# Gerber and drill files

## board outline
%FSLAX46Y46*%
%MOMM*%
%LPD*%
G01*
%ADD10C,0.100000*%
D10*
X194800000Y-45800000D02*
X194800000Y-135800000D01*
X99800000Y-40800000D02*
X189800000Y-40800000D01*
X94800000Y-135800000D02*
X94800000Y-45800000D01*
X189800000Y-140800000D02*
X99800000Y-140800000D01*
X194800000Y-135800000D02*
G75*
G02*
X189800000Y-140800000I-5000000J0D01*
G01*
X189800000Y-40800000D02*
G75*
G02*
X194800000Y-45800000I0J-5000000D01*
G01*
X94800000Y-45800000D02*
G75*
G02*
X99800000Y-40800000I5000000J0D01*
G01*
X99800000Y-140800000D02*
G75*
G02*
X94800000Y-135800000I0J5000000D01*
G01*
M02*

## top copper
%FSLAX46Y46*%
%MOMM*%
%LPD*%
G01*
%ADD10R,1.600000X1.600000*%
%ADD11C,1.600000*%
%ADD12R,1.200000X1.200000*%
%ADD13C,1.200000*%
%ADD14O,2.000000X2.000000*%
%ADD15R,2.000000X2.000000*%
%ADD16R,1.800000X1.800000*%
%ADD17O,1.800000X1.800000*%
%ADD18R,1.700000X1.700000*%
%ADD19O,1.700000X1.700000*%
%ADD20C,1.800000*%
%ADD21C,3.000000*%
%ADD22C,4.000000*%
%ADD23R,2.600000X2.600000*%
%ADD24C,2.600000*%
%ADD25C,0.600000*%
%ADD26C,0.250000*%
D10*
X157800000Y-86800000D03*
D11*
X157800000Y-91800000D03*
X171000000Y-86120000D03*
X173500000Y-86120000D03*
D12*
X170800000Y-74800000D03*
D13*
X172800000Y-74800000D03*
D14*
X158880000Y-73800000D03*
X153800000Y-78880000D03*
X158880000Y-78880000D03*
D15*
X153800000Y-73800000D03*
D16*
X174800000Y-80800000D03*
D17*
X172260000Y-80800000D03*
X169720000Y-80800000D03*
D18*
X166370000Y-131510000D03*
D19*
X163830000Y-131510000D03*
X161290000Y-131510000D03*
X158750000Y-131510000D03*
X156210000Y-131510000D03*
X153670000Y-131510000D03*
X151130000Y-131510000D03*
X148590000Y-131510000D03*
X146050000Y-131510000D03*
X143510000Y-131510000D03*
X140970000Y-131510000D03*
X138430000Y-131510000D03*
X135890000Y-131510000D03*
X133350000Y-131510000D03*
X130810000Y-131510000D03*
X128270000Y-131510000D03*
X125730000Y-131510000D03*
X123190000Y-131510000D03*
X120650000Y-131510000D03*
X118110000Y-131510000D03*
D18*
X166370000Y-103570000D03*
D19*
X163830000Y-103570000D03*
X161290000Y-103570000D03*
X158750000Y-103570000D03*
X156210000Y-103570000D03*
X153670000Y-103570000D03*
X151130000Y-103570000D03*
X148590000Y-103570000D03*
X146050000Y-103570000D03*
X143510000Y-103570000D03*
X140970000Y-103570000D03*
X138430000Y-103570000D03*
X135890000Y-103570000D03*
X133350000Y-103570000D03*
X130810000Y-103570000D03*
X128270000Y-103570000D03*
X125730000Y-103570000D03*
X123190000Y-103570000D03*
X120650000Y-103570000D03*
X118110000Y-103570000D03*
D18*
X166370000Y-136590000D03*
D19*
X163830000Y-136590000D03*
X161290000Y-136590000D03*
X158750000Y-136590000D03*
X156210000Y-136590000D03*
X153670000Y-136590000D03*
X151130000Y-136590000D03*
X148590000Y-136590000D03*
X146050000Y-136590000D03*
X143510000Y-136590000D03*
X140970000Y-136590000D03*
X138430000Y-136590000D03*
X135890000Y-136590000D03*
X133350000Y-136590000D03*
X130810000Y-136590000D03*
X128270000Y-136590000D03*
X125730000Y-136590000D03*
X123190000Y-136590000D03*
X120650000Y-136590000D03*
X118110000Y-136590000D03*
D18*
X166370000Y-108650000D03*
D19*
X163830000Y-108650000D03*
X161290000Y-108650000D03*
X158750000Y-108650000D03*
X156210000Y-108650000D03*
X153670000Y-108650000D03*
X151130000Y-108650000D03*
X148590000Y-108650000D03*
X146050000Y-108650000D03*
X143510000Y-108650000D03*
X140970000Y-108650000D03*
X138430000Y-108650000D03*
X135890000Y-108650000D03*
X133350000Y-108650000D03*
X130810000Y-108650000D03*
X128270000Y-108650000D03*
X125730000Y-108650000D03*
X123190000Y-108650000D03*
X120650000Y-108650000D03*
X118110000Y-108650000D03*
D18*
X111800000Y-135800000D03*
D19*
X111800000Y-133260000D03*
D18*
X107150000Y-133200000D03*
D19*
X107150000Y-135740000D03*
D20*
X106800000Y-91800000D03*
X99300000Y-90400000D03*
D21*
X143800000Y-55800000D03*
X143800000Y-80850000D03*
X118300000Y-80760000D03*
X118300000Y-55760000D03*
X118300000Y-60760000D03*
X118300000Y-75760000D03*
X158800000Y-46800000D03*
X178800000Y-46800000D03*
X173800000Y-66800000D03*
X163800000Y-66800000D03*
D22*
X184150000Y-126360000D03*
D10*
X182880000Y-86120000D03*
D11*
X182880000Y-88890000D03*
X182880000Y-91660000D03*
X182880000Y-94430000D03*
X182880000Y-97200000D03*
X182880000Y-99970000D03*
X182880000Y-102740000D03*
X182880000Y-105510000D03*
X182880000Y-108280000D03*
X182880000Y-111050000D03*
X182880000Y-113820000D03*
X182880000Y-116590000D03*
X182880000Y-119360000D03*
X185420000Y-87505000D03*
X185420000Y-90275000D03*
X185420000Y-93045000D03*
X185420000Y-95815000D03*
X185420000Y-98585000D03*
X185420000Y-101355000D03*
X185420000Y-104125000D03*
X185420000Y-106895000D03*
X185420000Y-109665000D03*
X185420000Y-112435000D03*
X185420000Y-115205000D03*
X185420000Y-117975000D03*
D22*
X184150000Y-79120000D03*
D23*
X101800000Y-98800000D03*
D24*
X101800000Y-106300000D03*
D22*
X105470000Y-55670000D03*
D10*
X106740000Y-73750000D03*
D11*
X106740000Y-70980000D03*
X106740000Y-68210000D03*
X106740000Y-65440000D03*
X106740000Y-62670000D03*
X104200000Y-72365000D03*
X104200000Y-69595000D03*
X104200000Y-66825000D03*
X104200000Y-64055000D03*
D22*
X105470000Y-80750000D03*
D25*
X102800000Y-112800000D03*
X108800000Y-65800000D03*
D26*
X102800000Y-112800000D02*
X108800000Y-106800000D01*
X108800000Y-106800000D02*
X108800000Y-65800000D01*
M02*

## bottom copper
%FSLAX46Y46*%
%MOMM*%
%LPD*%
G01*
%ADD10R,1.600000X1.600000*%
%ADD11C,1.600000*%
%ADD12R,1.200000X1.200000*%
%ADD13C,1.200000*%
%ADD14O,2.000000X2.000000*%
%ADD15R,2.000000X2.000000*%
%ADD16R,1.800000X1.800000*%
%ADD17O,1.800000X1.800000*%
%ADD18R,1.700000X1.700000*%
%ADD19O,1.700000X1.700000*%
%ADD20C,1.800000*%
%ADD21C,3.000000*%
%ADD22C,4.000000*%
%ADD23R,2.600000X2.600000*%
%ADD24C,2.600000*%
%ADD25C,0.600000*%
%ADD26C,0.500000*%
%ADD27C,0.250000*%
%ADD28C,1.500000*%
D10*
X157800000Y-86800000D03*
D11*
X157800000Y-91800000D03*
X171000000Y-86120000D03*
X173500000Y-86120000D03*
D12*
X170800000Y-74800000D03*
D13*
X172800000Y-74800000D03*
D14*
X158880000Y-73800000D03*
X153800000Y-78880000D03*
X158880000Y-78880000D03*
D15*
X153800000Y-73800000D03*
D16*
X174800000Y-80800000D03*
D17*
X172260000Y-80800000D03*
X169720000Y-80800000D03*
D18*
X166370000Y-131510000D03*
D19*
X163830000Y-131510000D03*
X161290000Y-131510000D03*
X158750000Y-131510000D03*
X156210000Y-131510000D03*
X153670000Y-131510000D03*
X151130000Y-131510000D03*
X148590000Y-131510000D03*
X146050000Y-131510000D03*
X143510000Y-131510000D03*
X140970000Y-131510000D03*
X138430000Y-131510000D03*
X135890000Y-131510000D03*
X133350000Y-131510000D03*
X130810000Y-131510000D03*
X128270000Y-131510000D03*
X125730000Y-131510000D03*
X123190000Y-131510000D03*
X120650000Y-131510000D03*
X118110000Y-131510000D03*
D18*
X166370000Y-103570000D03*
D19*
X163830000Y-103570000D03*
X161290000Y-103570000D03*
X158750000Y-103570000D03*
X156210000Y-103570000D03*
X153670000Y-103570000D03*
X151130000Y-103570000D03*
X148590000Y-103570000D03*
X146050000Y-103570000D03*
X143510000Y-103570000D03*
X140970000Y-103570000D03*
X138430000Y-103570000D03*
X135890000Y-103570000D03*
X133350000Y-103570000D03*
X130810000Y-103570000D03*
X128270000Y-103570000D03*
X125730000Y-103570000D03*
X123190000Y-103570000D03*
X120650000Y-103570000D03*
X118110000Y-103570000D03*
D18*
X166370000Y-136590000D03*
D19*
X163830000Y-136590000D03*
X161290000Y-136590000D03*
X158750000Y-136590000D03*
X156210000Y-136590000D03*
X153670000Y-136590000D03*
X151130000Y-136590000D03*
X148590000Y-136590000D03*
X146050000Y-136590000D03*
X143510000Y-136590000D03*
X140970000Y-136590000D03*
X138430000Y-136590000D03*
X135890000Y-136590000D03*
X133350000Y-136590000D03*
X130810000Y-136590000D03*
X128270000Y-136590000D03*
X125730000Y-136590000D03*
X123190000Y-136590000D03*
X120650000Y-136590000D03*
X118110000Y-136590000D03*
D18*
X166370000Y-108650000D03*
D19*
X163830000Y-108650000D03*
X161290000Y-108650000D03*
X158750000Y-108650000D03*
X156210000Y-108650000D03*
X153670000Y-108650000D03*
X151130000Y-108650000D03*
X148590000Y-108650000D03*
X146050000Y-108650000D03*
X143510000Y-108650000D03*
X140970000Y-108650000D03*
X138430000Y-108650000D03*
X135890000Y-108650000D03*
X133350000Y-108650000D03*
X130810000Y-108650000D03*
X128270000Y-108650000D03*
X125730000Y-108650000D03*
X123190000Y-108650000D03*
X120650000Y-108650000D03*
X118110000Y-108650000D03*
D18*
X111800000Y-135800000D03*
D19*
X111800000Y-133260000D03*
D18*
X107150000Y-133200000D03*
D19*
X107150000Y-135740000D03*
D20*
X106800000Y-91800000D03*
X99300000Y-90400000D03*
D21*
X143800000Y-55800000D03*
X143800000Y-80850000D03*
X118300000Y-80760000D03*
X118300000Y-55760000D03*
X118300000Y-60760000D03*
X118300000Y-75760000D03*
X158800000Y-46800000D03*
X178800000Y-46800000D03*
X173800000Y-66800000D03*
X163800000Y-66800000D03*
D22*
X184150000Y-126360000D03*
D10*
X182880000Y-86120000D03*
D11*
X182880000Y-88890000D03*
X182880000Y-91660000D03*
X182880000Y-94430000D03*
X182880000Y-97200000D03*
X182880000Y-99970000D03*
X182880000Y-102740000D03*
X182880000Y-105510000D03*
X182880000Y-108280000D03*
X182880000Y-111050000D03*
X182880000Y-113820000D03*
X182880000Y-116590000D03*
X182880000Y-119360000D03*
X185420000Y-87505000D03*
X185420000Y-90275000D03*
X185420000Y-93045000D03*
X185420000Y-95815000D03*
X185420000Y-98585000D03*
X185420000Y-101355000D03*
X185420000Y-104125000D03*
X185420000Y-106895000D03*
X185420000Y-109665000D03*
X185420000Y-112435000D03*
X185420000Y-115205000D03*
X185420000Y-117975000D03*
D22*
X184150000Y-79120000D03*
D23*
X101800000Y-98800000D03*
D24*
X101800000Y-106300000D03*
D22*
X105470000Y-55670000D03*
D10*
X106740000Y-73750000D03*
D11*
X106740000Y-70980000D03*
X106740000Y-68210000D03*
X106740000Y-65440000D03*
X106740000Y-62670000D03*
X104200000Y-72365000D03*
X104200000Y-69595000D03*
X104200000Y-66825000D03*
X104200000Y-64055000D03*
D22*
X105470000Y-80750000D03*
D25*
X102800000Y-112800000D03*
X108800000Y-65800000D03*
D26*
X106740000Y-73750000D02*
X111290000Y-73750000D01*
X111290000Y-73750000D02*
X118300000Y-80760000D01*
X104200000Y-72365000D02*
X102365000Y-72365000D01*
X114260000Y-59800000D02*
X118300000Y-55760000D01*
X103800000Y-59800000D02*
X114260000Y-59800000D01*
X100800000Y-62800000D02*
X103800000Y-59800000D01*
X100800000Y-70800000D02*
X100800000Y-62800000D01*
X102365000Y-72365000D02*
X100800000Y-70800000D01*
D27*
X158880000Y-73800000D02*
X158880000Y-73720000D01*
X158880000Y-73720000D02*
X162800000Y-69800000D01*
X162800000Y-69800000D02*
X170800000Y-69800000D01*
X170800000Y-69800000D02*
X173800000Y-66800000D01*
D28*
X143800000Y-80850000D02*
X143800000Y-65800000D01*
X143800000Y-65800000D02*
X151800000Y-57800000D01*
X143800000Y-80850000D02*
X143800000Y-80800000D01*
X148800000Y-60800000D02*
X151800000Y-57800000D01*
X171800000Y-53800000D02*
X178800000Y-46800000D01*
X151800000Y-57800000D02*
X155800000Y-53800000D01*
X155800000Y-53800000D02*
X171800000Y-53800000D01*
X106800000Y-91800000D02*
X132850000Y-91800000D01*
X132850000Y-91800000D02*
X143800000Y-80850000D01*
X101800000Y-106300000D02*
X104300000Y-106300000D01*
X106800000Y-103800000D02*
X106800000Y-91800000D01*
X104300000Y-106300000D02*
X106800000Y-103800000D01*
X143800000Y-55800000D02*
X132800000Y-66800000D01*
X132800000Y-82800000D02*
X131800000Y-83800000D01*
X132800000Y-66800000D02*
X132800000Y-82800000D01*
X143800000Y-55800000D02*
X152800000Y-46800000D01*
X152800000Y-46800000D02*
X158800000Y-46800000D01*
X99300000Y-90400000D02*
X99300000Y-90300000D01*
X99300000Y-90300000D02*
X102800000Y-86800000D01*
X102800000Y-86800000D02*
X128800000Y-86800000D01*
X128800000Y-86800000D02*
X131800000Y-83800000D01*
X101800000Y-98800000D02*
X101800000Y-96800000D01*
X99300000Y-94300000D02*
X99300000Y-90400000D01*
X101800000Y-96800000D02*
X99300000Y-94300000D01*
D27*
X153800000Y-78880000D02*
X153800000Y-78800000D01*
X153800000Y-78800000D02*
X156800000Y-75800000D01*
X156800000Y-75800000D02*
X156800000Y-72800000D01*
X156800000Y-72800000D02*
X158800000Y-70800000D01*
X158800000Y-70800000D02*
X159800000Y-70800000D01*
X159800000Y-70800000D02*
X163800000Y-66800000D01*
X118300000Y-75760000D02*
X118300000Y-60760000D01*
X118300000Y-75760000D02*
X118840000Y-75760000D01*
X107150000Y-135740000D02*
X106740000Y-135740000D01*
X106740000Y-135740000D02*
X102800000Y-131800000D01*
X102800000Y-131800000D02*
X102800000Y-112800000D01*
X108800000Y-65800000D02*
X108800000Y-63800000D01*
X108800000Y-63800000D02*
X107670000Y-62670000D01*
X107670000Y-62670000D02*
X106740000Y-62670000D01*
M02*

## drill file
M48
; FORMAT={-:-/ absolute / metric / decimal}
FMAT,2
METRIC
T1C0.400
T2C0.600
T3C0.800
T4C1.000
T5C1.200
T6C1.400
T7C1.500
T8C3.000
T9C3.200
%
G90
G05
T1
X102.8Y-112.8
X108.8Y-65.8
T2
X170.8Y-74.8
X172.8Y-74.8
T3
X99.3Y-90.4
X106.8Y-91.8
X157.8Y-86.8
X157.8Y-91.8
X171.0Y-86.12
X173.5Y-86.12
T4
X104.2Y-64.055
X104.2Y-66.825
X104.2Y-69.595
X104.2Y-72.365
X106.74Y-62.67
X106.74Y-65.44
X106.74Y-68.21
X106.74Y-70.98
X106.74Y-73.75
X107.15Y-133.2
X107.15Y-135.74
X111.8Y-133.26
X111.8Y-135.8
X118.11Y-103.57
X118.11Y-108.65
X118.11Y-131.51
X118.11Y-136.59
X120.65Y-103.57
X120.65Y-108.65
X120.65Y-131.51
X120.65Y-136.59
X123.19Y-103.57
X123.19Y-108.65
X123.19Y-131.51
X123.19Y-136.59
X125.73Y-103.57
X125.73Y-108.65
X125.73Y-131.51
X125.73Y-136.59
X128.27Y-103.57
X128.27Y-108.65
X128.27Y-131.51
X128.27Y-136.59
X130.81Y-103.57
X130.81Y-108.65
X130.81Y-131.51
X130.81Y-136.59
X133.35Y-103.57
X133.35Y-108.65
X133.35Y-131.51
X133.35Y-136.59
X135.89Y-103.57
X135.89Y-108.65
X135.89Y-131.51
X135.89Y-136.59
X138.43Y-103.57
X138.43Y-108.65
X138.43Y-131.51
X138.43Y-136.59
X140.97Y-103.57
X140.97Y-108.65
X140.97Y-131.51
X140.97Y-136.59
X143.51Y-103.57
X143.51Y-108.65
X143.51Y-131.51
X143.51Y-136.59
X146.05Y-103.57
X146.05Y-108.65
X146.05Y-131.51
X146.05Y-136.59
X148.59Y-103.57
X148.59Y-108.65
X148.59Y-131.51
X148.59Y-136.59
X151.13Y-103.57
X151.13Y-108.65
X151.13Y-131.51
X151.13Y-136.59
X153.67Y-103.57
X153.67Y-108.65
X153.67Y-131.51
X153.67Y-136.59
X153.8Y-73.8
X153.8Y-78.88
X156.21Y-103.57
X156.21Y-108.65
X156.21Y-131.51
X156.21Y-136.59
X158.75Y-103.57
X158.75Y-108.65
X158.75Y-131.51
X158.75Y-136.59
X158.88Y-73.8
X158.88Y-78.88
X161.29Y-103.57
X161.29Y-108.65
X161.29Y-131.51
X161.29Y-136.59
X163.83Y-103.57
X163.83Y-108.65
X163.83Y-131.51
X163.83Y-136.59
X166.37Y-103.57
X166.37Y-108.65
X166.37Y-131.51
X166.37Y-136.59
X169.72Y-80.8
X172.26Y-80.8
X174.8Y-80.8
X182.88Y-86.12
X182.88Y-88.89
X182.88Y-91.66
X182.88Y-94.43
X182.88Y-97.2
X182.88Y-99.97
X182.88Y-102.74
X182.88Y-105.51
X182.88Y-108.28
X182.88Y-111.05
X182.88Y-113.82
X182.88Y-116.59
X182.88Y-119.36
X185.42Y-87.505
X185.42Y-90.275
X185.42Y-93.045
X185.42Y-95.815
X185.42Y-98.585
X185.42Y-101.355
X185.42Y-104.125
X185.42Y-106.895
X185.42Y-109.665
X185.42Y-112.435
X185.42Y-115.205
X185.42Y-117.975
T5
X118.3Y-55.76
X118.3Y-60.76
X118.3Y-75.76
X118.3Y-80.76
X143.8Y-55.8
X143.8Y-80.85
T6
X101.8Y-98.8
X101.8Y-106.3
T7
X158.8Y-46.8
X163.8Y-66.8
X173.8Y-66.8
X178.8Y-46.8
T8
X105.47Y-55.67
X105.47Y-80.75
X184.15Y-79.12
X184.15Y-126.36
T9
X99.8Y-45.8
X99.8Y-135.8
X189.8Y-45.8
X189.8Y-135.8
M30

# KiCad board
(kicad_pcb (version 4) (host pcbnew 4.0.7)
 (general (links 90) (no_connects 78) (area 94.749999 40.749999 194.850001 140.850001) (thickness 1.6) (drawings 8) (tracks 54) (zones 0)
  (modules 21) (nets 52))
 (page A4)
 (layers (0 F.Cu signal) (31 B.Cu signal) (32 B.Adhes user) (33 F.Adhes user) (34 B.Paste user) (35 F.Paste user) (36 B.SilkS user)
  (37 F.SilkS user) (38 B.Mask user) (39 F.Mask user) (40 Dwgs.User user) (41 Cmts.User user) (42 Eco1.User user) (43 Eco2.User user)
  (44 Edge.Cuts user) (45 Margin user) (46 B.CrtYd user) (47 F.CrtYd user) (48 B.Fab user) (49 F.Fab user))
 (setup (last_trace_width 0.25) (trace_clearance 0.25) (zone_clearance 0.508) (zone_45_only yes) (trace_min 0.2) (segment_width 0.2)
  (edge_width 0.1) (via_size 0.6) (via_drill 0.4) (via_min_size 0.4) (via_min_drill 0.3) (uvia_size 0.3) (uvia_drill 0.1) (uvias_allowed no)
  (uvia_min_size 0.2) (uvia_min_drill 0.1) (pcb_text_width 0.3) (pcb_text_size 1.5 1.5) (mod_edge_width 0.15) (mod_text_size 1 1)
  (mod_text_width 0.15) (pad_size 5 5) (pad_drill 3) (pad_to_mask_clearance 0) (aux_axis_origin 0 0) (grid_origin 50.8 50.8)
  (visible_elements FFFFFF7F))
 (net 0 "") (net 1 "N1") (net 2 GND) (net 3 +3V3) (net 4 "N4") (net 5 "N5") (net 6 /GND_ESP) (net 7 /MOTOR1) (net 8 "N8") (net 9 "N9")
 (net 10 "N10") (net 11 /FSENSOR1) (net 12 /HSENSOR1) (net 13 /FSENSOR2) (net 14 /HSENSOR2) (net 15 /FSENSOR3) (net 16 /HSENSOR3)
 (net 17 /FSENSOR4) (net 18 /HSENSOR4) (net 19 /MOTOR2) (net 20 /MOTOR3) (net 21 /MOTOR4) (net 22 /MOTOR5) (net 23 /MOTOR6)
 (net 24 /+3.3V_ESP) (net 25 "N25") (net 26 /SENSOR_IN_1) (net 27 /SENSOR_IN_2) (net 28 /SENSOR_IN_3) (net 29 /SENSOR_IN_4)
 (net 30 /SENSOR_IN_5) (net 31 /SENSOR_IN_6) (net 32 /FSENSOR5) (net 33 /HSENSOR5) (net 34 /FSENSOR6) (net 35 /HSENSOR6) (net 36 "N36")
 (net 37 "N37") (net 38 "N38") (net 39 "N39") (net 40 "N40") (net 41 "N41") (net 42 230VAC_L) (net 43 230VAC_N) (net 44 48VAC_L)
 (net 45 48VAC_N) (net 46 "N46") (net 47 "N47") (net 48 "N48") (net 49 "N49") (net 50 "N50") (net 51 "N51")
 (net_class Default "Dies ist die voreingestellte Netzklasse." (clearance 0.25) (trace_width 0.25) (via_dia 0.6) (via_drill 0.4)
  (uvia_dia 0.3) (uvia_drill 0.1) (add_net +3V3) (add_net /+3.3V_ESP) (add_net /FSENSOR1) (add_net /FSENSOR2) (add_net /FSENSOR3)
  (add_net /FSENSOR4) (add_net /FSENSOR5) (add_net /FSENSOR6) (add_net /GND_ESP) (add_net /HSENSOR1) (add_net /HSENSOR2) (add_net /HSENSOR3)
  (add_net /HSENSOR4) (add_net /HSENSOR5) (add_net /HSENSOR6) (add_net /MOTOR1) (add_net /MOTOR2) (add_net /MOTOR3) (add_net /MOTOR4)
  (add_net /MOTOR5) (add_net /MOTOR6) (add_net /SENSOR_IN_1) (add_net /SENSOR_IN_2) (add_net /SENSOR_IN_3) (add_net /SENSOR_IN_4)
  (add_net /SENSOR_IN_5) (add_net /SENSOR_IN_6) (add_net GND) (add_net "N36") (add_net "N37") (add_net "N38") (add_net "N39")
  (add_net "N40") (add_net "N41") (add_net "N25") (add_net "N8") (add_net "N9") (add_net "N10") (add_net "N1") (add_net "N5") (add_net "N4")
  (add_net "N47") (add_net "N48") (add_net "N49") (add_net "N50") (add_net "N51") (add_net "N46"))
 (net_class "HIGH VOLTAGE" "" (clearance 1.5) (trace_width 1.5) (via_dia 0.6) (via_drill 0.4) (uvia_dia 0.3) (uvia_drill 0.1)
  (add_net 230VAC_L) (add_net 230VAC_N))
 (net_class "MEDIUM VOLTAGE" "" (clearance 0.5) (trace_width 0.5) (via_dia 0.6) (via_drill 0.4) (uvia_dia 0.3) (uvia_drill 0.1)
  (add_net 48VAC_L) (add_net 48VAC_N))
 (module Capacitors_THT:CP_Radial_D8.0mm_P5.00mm (layer F.Cu) (at 157.8 86.8 270)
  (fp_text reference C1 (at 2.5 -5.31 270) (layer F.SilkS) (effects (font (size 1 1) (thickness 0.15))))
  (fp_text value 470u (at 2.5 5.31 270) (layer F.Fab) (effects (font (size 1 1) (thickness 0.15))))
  (pad 1 thru_hole rect (at 0 0 270) (size 1.6 1.6) (drill 0.8) (layers *.Cu *.Mask) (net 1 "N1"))
  (pad 2 thru_hole circle (at 5 0 270) (size 1.6 1.6) (drill 0.8) (layers *.Cu *.Mask) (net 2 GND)))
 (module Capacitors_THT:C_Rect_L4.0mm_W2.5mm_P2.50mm (layer F.Cu) (at 171 86.12)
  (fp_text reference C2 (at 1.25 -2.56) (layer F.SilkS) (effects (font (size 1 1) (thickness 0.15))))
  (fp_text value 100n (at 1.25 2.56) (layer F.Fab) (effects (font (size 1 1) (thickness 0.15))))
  (pad 1 thru_hole circle (at 0 0) (size 1.6 1.6) (drill 0.8) (layers *.Cu *.Mask) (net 1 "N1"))
  (pad 2 thru_hole circle (at 2.5 0) (size 1.6 1.6) (drill 0.8) (layers *.Cu *.Mask) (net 2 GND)))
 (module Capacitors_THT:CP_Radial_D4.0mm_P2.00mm (layer F.Cu) (at 170.8 74.8)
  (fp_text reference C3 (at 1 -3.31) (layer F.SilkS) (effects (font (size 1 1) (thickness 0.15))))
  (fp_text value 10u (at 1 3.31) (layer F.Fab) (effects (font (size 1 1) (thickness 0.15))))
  (pad 1 thru_hole rect (at 0 0) (size 1.2 1.2) (drill 0.6) (layers *.Cu *.Mask) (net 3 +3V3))
  (pad 2 thru_hole circle (at 2 0) (size 1.2 1.2) (drill 0.6) (layers *.Cu *.Mask) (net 2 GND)))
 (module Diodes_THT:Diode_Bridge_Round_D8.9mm (layer F.Cu) (at 153.8 73.8)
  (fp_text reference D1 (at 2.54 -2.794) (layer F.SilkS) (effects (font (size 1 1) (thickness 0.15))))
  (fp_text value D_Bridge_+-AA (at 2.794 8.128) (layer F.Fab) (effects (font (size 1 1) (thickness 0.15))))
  (pad 4 thru_hole oval (at 5.08 0) (size 2 2) (drill 1) (layers *.Cu *.Mask) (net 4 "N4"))
  (pad 2 thru_hole oval (at 0 5.08) (size 2 2) (drill 1) (layers *.Cu *.Mask) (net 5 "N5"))
  (pad 3 thru_hole oval (at 5.08 5.08) (size 2 2) (drill 1) (layers *.Cu *.Mask) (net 2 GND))
  (pad 1 thru_hole rect (at 0 0) (size 2 2) (drill 1) (layers *.Cu *.Mask) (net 1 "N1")))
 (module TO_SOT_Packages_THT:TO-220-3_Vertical (layer F.Cu) (at 174.8 80.8 180)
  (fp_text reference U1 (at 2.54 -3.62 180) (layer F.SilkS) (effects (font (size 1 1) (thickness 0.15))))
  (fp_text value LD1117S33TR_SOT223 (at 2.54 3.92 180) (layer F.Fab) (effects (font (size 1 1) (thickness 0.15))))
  (pad 1 thru_hole rect (at 0 0 180) (size 1.8 1.8) (drill 1) (layers *.Cu *.Mask) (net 2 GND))
  (pad 2 thru_hole oval (at 2.54 0 180) (size 1.8 1.8) (drill 1) (layers *.Cu *.Mask) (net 3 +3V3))
  (pad 3 thru_hole oval (at 5.08 0 180) (size 1.8 1.8) (drill 1) (layers *.Cu *.Mask) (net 1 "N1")))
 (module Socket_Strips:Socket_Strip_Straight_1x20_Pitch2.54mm (layer F.Cu) (at 166.37 131.51 270)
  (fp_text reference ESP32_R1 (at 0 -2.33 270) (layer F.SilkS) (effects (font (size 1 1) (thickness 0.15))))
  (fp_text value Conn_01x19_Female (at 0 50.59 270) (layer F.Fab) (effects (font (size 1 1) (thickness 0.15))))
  (pad 1 thru_hole rect (at 0 0 270) (size 1.7 1.7) (drill 1) (layers *.Cu *.Mask) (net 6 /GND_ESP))
  (pad 2 thru_hole oval (at 0 2.54 270) (size 1.7 1.7) (drill 1) (layers *.Cu *.Mask) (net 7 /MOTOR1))
  (pad 3 thru_hole oval (at 0 5.08 270) (size 1.7 1.7) (drill 1) (layers *.Cu *.Mask) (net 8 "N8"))
  (pad 4 thru_hole oval (at 0 7.62 270) (size 1.7 1.7) (drill 1) (layers *.Cu *.Mask) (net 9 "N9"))
  (pad 5 thru_hole oval (at 0 10.16 270) (size 1.7 1.7) (drill 1) (layers *.Cu *.Mask) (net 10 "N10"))
  (pad 6 thru_hole oval (at 0 12.7 270) (size 1.7 1.7) (drill 1) (layers *.Cu *.Mask) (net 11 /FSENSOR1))
  (pad 7 thru_hole oval (at 0 15.24 270) (size 1.7 1.7) (drill 1) (layers *.Cu *.Mask) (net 6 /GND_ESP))
  (pad 8 thru_hole oval (at 0 17.78 270) (size 1.7 1.7) (drill 1) (layers *.Cu *.Mask) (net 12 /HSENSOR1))
  (pad 9 thru_hole oval (at 0 20.32 270) (size 1.7 1.7) (drill 1) (layers *.Cu *.Mask) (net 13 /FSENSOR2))
  (pad 10 thru_hole oval (at 0 22.86 270) (size 1.7 1.7) (drill 1) (layers *.Cu *.Mask) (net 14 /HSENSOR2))
  (pad 11 thru_hole oval (at 0 25.4 270) (size 1.7 1.7) (drill 1) (layers *.Cu *.Mask) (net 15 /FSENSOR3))
  (pad 12 thru_hole oval (at 0 27.94 270) (size 1.7 1.7) (drill 1) (layers *.Cu *.Mask) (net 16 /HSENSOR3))
  (pad 13 thru_hole oval (at 0 30.48 270) (size 1.7 1.7) (drill 1) (layers *.Cu *.Mask) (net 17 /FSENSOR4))
  (pad 14 thru_hole oval (at 0 33.02 270) (size 1.7 1.7) (drill 1) (layers *.Cu *.Mask) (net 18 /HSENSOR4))
  (pad 15 thru_hole oval (at 0 35.56 270) (size 1.7 1.7) (drill 1) (layers *.Cu *.Mask) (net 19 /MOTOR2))
  (pad 16 thru_hole oval (at 0 38.1 270) (size 1.7 1.7) (drill 1) (layers *.Cu *.Mask) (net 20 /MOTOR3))
  (pad 17 thru_hole oval (at 0 40.64 270) (size 1.7 1.7) (drill 1) (layers *.Cu *.Mask) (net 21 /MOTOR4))
  (pad 18 thru_hole oval (at 0 43.18 270) (size 1.7 1.7) (drill 1) (layers *.Cu *.Mask) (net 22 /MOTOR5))
  (pad 19 thru_hole oval (at 0 45.72 270) (size 1.7 1.7) (drill 1) (layers *.Cu *.Mask) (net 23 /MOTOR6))
  (pad 20 thru_hole oval (at 0 48.26 270) (size 1.7 1.7) (drill 1) (layers *.Cu *.Mask)))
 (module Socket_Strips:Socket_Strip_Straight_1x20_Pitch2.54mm (layer F.Cu) (at 166.37 103.57 270)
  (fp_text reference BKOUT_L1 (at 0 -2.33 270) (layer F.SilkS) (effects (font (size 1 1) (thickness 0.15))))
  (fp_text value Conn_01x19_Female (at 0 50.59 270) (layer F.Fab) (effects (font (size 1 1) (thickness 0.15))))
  (pad 1 thru_hole rect (at 0 0 270) (size 1.7 1.7) (drill 1) (layers *.Cu *.Mask) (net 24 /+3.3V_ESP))
  (pad 2 thru_hole oval (at 0 2.54 270) (size 1.7 1.7) (drill 1) (layers *.Cu *.Mask) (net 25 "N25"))
  (pad 3 thru_hole oval (at 0 5.08 270) (size 1.7 1.7) (drill 1) (layers *.Cu *.Mask) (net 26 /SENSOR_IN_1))
  (pad 4 thru_hole oval (at 0 7.62 270) (size 1.7 1.7) (drill 1) (layers *.Cu *.Mask) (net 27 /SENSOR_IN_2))
  (pad 5 thru_hole oval (at 0 10.16 270) (size 1.7 1.7) (drill 1) (layers *.Cu *.Mask) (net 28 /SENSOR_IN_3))
  (pad 6 thru_hole oval (at 0 12.7 270) (size 1.7 1.7) (drill 1) (layers *.Cu *.Mask) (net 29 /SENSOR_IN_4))
  (pad 7 thru_hole oval (at 0 15.24 270) (size 1.7 1.7) (drill 1) (layers *.Cu *.Mask) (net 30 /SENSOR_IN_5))
  (pad 8 thru_hole oval (at 0 17.78 270) (size 1.7 1.7) (drill 1) (layers *.Cu *.Mask) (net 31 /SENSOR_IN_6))
  (pad 9 thru_hole oval (at 0 20.32 270) (size 1.7 1.7) (drill 1) (layers *.Cu *.Mask) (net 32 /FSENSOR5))
  (pad 10 thru_hole oval (at 0 22.86 270) (size 1.7 1.7) (drill 1) (layers *.Cu *.Mask) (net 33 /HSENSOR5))
  (pad 11 thru_hole oval (at 0 25.4 270) (size 1.7 1.7) (drill 1) (layers *.Cu *.Mask) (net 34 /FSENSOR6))
  (pad 12 thru_hole oval (at 0 27.94 270) (size 1.7 1.7) (drill 1) (layers *.Cu *.Mask) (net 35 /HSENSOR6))
  (pad 13 thru_hole oval (at 0 30.48 270) (size 1.7 1.7) (drill 1) (layers *.Cu *.Mask) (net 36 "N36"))
  (pad 14 thru_hole oval (at 0 33.02 270) (size 1.7 1.7) (drill 1) (layers *.Cu *.Mask) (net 6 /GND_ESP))
  (pad 15 thru_hole oval (at 0 35.56 270) (size 1.7 1.7) (drill 1) (layers *.Cu *.Mask) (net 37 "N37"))
  (pad 16 thru_hole oval (at 0 38.1 270) (size 1.7 1.7) (drill 1) (layers *.Cu *.Mask) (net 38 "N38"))
  (pad 17 thru_hole oval (at 0 40.64 270) (size 1.7 1.7) (drill 1) (layers *.Cu *.Mask) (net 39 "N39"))
  (pad 18 thru_hole oval (at 0 43.18 270) (size 1.7 1.7) (drill 1) (layers *.Cu *.Mask) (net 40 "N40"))
  (pad 19 thru_hole oval (at 0 45.72 270) (size 1.7 1.7) (drill 1) (layers *.Cu *.Mask) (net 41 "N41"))
  (pad 20 thru_hole oval (at 0 48.26 270) (size 1.7 1.7) (drill 1) (layers *.Cu *.Mask)))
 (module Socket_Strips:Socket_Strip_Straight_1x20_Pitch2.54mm (layer F.Cu) (at 166.37 136.59 270)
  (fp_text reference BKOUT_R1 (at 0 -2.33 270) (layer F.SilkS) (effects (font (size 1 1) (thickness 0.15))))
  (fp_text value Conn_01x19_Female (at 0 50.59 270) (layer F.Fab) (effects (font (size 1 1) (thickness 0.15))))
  (pad 1 thru_hole rect (at 0 0 270) (size 1.7 1.7) (drill 1) (layers *.Cu *.Mask) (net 6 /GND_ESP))
  (pad 2 thru_hole oval (at 0 2.54 270) (size 1.7 1.7) (drill 1) (layers *.Cu *.Mask) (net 7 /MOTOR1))
  (pad 3 thru_hole oval (at 0 5.08 270) (size 1.7 1.7) (drill 1) (layers *.Cu *.Mask) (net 8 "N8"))
  (pad 4 thru_hole oval (at 0 7.62 270) (size 1.7 1.7) (drill 1) (layers *.Cu *.Mask) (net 9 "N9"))
  (pad 5 thru_hole oval (at 0 10.16 270) (size 1.7 1.7) (drill 1) (layers *.Cu *.Mask) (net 10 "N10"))
  (pad 6 thru_hole oval (at 0 12.7 270) (size 1.7 1.7) (drill 1) (layers *.Cu *.Mask) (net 11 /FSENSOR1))
  (pad 7 thru_hole oval (at 0 15.24 270) (size 1.7 1.7) (drill 1) (layers *.Cu *.Mask) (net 6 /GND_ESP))
  (pad 8 thru_hole oval (at 0 17.78 270) (size 1.7 1.7) (drill 1) (layers *.Cu *.Mask) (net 12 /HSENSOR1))
  (pad 9 thru_hole oval (at 0 20.32 270) (size 1.7 1.7) (drill 1) (layers *.Cu *.Mask) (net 13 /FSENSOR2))
  (pad 10 thru_hole oval (at 0 22.86 270) (size 1.7 1.7) (drill 1) (layers *.Cu *.Mask) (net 14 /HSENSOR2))
  (pad 11 thru_hole oval (at 0 25.4 270) (size 1.7 1.7) (drill 1) (layers *.Cu *.Mask) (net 15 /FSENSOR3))
  (pad 12 thru_hole oval (at 0 27.94 270) (size 1.7 1.7) (drill 1) (layers *.Cu *.Mask) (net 16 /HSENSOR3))
  (pad 13 thru_hole oval (at 0 30.48 270) (size 1.7 1.7) (drill 1) (layers *.Cu *.Mask) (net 17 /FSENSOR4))
  (pad 14 thru_hole oval (at 0 33.02 270) (size 1.7 1.7) (drill 1) (layers *.Cu *.Mask) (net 18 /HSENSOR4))
  (pad 15 thru_hole oval (at 0 35.56 270) (size 1.7 1.7) (drill 1) (layers *.Cu *.Mask) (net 19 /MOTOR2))
  (pad 16 thru_hole oval (at 0 38.1 270) (size 1.7 1.7) (drill 1) (layers *.Cu *.Mask) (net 20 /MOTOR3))
  (pad 17 thru_hole oval (at 0 40.64 270) (size 1.7 1.7) (drill 1) (layers *.Cu *.Mask) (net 21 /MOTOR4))
  (pad 18 thru_hole oval (at 0 43.18 270) (size 1.7 1.7) (drill 1) (layers *.Cu *.Mask) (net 22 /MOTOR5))
  (pad 19 thru_hole oval (at 0 45.72 270) (size 1.7 1.7) (drill 1) (layers *.Cu *.Mask) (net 23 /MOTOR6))
  (pad 20 thru_hole oval (at 0 48.26 270) (size 1.7 1.7) (drill 1) (layers *.Cu *.Mask)))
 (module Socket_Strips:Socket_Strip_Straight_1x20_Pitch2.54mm (layer F.Cu) (at 166.37 108.65 270)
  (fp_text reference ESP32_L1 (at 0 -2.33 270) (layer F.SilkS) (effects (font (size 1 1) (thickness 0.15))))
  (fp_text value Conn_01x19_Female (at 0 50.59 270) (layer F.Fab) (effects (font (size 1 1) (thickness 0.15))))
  (pad 1 thru_hole rect (at 0 0 270) (size 1.7 1.7) (drill 1) (layers *.Cu *.Mask) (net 24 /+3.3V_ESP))
  (pad 2 thru_hole oval (at 0 2.54 270) (size 1.7 1.7) (drill 1) (layers *.Cu *.Mask) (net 25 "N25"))
  (pad 3 thru_hole oval (at 0 5.08 270) (size 1.7 1.7) (drill 1) (layers *.Cu *.Mask) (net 26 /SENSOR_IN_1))
  (pad 4 thru_hole oval (at 0 7.62 270) (size 1.7 1.7) (drill 1) (layers *.Cu *.Mask) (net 27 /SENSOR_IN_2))
  (pad 5 thru_hole oval (at 0 10.16 270) (size 1.7 1.7) (drill 1) (layers *.Cu *.Mask) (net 28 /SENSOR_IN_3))
  (pad 6 thru_hole oval (at 0 12.7 270) (size 1.7 1.7) (drill 1) (layers *.Cu *.Mask) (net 29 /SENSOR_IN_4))
  (pad 7 thru_hole oval (at 0 15.24 270) (size 1.7 1.7) (drill 1) (layers *.Cu *.Mask) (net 30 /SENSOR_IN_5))
  (pad 8 thru_hole oval (at 0 17.78 270) (size 1.7 1.7) (drill 1) (layers *.Cu *.Mask) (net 31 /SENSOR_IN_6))
  (pad 9 thru_hole oval (at 0 20.32 270) (size 1.7 1.7) (drill 1) (layers *.Cu *.Mask) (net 32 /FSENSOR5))
  (pad 10 thru_hole oval (at 0 22.86 270) (size 1.7 1.7) (drill 1) (layers *.Cu *.Mask) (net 33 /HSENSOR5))
  (pad 11 thru_hole oval (at 0 25.4 270) (size 1.7 1.7) (drill 1) (layers *.Cu *.Mask) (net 34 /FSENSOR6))
  (pad 12 thru_hole oval (at 0 27.94 270) (size 1.7 1.7) (drill 1) (layers *.Cu *.Mask) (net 35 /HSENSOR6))
  (pad 13 thru_hole oval (at 0 30.48 270) (size 1.7 1.7) (drill 1) (layers *.Cu *.Mask) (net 36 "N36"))
  (pad 14 thru_hole oval (at 0 33.02 270) (size 1.7 1.7) (drill 1) (layers *.Cu *.Mask) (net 6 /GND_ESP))
  (pad 15 thru_hole oval (at 0 35.56 270) (size 1.7 1.7) (drill 1) (layers *.Cu *.Mask) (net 37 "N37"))
  (pad 16 thru_hole oval (at 0 38.1 270) (size 1.7 1.7) (drill 1) (layers *.Cu *.Mask) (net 38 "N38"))
  (pad 17 thru_hole oval (at 0 40.64 270) (size 1.7 1.7) (drill 1) (layers *.Cu *.Mask) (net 39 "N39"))
  (pad 18 thru_hole oval (at 0 43.18 270) (size 1.7 1.7) (drill 1) (layers *.Cu *.Mask) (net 40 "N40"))
  (pad 19 thru_hole oval (at 0 45.72 270) (size 1.7 1.7) (drill 1) (layers *.Cu *.Mask) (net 41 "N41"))
  (pad 20 thru_hole oval (at 0 48.26 270) (size 1.7 1.7) (drill 1) (layers *.Cu *.Mask)))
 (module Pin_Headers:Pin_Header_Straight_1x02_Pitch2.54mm (layer F.Cu) (at 111.8 135.8 180)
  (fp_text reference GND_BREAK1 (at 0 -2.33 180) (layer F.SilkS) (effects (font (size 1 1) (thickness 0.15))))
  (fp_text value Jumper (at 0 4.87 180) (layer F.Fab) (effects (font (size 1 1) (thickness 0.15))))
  (pad 1 thru_hole rect (at 0 0 180) (size 1.7 1.7) (drill 1) (layers *.Cu *.Mask) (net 2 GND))
  (pad 2 thru_hole oval (at 0 2.54 180) (size 1.7 1.7) (drill 1) (layers *.Cu *.Mask) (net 6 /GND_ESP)))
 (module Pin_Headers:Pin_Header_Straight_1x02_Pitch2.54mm (layer F.Cu) (at 107.15 133.2)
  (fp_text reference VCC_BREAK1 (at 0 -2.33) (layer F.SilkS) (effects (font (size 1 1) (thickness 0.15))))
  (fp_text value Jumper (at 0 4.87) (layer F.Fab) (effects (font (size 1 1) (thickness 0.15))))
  (pad 1 thru_hole rect (at 0 0) (size 1.7 1.7) (drill 1) (layers *.Cu *.Mask) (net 3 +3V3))
  (pad 2 thru_hole oval (at 0 2.54) (size 1.7 1.7) (drill 1) (layers *.Cu *.Mask) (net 24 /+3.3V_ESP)))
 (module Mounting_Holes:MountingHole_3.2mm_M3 (layer F.Cu) (at 99.8 135.8)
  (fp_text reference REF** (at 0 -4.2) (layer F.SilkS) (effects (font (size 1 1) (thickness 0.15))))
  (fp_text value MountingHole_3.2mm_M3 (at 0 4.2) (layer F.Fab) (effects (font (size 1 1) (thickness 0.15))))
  (pad 1 np_thru_hole circle (at 0 0) (size 3.2 3.2) (drill 3.2) (layers *.Cu *.Mask)))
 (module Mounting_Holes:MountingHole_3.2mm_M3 (layer F.Cu) (at 99.8 45.8)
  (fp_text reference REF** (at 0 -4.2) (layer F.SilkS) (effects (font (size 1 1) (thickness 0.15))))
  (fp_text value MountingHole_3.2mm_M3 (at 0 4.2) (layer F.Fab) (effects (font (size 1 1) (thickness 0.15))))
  (pad 1 np_thru_hole circle (at 0 0) (size 3.2 3.2) (drill 3.2) (layers *.Cu *.Mask)))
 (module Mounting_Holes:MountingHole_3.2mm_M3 (layer F.Cu) (at 189.8 45.8)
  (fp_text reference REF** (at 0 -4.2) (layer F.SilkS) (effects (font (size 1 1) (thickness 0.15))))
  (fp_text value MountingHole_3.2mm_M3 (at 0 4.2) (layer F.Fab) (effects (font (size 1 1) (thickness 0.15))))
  (pad 1 np_thru_hole circle (at 0 0) (size 3.2 3.2) (drill 3.2) (layers *.Cu *.Mask)))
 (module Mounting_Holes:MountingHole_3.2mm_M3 (layer F.Cu) (at 189.8 135.8)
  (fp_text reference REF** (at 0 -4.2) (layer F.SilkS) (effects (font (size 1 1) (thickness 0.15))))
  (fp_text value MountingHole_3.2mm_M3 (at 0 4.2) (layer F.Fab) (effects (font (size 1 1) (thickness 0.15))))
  (pad 1 np_thru_hole circle (at 0 0) (size 3.2 3.2) (drill 3.2) (layers *.Cu *.Mask)))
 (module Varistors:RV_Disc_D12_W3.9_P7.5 (layer F.Cu) (at 106.8 91.8 180)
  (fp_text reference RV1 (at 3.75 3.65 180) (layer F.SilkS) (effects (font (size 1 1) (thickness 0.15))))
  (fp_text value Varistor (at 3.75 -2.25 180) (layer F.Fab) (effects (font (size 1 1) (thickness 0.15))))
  (pad 1 thru_hole circle (at 0 0 180) (size 1.8 1.8) (drill 0.8) (layers *.Cu *.Mask) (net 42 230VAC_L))
  (pad 2 thru_hole circle (at 7.5 1.4 180) (size 1.8 1.8) (drill 0.8) (layers *.Cu *.Mask) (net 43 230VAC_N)))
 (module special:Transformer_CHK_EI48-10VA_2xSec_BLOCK (layer F.Cu) (at 143.8 55.8 180)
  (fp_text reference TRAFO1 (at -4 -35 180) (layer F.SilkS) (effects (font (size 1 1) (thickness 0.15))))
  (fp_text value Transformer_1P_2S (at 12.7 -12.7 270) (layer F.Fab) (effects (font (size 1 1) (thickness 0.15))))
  (pad 1 thru_hole circle (at 0 0 180) (size 3 3) (drill 1.2) (layers *.Cu *.Mask) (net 43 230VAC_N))
  (pad 6 thru_hole circle (at 0 -25.05 180) (size 3 3) (drill 1.2) (layers *.Cu *.Mask) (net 42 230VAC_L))
  (pad 7 thru_hole circle (at 25.5 -24.96 180) (size 3 3) (drill 1.2) (layers *.Cu *.Mask) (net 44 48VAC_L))
  (pad 12 thru_hole circle (at 25.5 0.04 180) (size 3 3) (drill 1.2) (layers *.Cu *.Mask) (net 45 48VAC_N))
  (pad 11 thru_hole circle (at 25.5 -4.96 180) (size 3 3) (drill 1.2) (layers *.Cu *.Mask) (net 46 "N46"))
  (pad 8 thru_hole circle (at 25.5 -19.96 180) (size 3 3) (drill 1.2) (layers *.Cu *.Mask) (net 46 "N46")))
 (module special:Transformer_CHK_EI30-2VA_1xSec (layer F.Cu) (at 158.8 46.8 270)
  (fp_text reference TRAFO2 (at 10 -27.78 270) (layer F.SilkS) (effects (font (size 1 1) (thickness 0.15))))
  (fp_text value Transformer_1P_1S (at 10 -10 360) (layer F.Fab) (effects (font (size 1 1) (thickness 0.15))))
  (pad 1 thru_hole circle (at 0 0 270) (size 3 3) (drill 1.5) (layers *.Cu *.Mask) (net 43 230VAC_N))
  (pad 5 thru_hole circle (at 0 -20 270) (size 3 3) (drill 1.5) (layers *.Cu *.Mask) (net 42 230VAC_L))
  (pad 7 thru_hole circle (at 20 -15 270) (size 3 3) (drill 1.5) (layers *.Cu *.Mask) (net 4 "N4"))
  (pad 9 thru_hole circle (at 20 -5 270) (size 3 3) (drill 1.5) (layers *.Cu *.Mask) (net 5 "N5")))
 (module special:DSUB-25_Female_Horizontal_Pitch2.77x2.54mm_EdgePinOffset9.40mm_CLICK (layer F.Cu) (at 182.88 86.12 90)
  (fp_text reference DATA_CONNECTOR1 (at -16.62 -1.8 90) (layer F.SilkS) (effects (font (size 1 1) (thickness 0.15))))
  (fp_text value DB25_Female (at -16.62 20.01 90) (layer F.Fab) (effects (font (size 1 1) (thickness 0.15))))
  (pad B1 thru_hole circle (at -40.24 1.27 90) (size 4 4) (drill 3) (layers *.Cu *.Mask))
  (pad 1 thru_hole rect (at 0 0 90) (size 1.6 1.6) (drill 1) (layers *.Cu *.Mask) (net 7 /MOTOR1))
  (pad 2 thru_hole circle (at -2.77 0 90) (size 1.6 1.6) (drill 1) (layers *.Cu *.Mask) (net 11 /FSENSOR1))
  (pad 3 thru_hole circle (at -5.54 0 90) (size 1.6 1.6) (drill 1) (layers *.Cu *.Mask) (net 19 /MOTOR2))
  (pad 4 thru_hole circle (at -8.31 0 90) (size 1.6 1.6) (drill 1) (layers *.Cu *.Mask) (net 13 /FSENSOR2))
  (pad 5 thru_hole circle (at -11.08 0 90) (size 1.6 1.6) (drill 1) (layers *.Cu *.Mask) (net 20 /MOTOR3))
  (pad 6 thru_hole circle (at -13.85 0 90) (size 1.6 1.6) (drill 1) (layers *.Cu *.Mask) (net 15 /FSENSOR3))
  (pad 7 thru_hole circle (at -16.62 0 90) (size 1.6 1.6) (drill 1) (layers *.Cu *.Mask) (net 21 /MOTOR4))
  (pad 8 thru_hole circle (at -19.39 0 90) (size 1.6 1.6) (drill 1) (layers *.Cu *.Mask) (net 17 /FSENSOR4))
  (pad 9 thru_hole circle (at -22.16 0 90) (size 1.6 1.6) (drill 1) (layers *.Cu *.Mask) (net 22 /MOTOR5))
  (pad 10 thru_hole circle (at -24.93 0 90) (size 1.6 1.6) (drill 1) (layers *.Cu *.Mask) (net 32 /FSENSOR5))
  (pad 11 thru_hole circle (at -27.7 0 90) (size 1.6 1.6) (drill 1) (layers *.Cu *.Mask) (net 23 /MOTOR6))
  (pad 12 thru_hole circle (at -30.47 0 90) (size 1.6 1.6) (drill 1) (layers *.Cu *.Mask) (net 34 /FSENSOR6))
  (pad 13 thru_hole circle (at -33.24 0 90) (size 1.6 1.6) (drill 1) (layers *.Cu *.Mask) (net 2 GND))
  (pad 14 thru_hole circle (at -1.385 2.54 90) (size 1.6 1.6) (drill 1) (layers *.Cu *.Mask) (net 26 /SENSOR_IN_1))
  (pad 15 thru_hole circle (at -4.155 2.54 90) (size 1.6 1.6) (drill 1) (layers *.Cu *.Mask) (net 12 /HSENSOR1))
  (pad 16 thru_hole circle (at -6.925 2.54 90) (size 1.6 1.6) (drill 1) (layers *.Cu *.Mask) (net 27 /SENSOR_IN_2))
  (pad 17 thru_hole circle (at -9.695 2.54 90) (size 1.6 1.6) (drill 1) (layers *.Cu *.Mask) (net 14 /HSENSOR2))
  (pad 18 thru_hole circle (at -12.465 2.54 90) (size 1.6 1.6) (drill 1) (layers *.Cu *.Mask) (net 28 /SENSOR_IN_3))
  (pad 19 thru_hole circle (at -15.235 2.54 90) (size 1.6 1.6) (drill 1) (layers *.Cu *.Mask) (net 16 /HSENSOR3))
  (pad 20 thru_hole circle (at -18.005 2.54 90) (size 1.6 1.6) (drill 1) (layers *.Cu *.Mask) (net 29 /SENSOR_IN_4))
  (pad 21 thru_hole circle (at -20.775 2.54 90) (size 1.6 1.6) (drill 1) (layers *.Cu *.Mask) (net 18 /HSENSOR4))
  (pad 22 thru_hole circle (at -23.545 2.54 90) (size 1.6 1.6) (drill 1) (layers *.Cu *.Mask) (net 30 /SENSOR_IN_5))
  (pad 23 thru_hole circle (at -26.315 2.54 90) (size 1.6 1.6) (drill 1) (layers *.Cu *.Mask) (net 33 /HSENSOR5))
  (pad 24 thru_hole circle (at -29.085 2.54 90) (size 1.6 1.6) (drill 1) (layers *.Cu *.Mask) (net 31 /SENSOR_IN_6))
  (pad 25 thru_hole circle (at -31.855 2.54 90) (size 1.6 1.6) (drill 1) (layers *.Cu *.Mask) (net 35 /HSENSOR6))
  (pad B2 thru_hole circle (at 7 1.27 90) (size 4 4) (drill 3) (layers *.Cu *.Mask)))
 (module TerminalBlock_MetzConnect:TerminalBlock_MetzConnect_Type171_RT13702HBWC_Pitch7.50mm (layer F.Cu) (at 101.8 98.8 270)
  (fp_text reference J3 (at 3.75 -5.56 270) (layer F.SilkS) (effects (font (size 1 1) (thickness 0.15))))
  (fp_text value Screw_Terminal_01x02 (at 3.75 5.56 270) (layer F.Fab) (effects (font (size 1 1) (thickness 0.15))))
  (pad 1 thru_hole rect (at 0 0 270) (size 2.6 2.6) (drill 1.4) (layers *.Cu *.Mask) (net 43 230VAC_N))
  (pad 2 thru_hole circle (at 7.5 0 270) (size 2.6 2.6) (drill 1.4) (layers *.Cu *.Mask) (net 42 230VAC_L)))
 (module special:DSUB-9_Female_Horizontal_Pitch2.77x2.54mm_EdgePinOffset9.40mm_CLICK (layer F.Cu) (at 106.74 73.75 270)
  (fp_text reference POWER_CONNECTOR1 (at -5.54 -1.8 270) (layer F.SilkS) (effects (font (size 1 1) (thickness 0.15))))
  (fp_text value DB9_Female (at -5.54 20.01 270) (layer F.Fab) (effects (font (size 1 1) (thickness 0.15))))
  (pad B1 thru_hole circle (at -18.08 1.27 270) (size 4 4) (drill 3) (layers *.Cu *.Mask))
  (pad 1 thru_hole rect (at 0 0 270) (size 1.6 1.6) (drill 1) (layers *.Cu *.Mask) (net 44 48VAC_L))
  (pad 2 thru_hole circle (at -2.77 0 270) (size 1.6 1.6) (drill 1) (layers *.Cu *.Mask) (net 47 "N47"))
  (pad 3 thru_hole circle (at -5.54 0 270) (size 1.6 1.6) (drill 1) (layers *.Cu *.Mask) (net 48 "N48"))
  (pad 4 thru_hole circle (at -8.31 0 270) (size 1.6 1.6) (drill 1) (layers *.Cu *.Mask) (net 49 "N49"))
  (pad 5 thru_hole circle (at -11.08 0 270) (size 1.6 1.6) (drill 1) (layers *.Cu *.Mask) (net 24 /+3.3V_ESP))
  (pad 6 thru_hole circle (at -1.385 2.54 270) (size 1.6 1.6) (drill 1) (layers *.Cu *.Mask) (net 45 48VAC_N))
  (pad 7 thru_hole circle (at -4.155 2.54 270) (size 1.6 1.6) (drill 1) (layers *.Cu *.Mask) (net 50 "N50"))
  (pad 8 thru_hole circle (at -6.925 2.54 270) (size 1.6 1.6) (drill 1) (layers *.Cu *.Mask) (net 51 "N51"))
  (pad 9 thru_hole circle (at -9.695 2.54 270) (size 1.6 1.6) (drill 1) (layers *.Cu *.Mask) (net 6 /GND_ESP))
  (pad B2 thru_hole circle (at 7 1.27 270) (size 4 4) (drill 3) (layers *.Cu *.Mask)))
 (gr_line (start 194.8 45.8) (end 194.8 135.8) (angle 90) (layer Edge.Cuts) (width 0.1))
 (gr_line (start 99.8 40.8) (end 189.8 40.8) (angle 90) (layer Edge.Cuts) (width 0.1))
 (gr_line (start 94.8 135.8) (end 94.8 45.8) (angle 90) (layer Edge.Cuts) (width 0.1))
 (gr_line (start 189.8 140.8) (end 99.8 140.8) (angle 90) (layer Edge.Cuts) (width 0.1))
 (gr_arc (start 189.8 135.8) (end 194.8 135.8) (angle 90) (layer Edge.Cuts) (width 0.1))
 (gr_arc (start 189.8 45.8) (end 189.8 40.8) (angle 90) (layer Edge.Cuts) (width 0.1))
 (gr_arc (start 99.8 45.8) (end 94.8 45.8) (angle 90) (layer Edge.Cuts) (width 0.1))
 (gr_arc (start 99.8 135.8) (end 99.8 140.8) (angle 90) (layer Edge.Cuts) (width 0.1))
 (segment (start 106.74 73.75) (end 111.29 73.75) (width 0.5) (layer B.Cu) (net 44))
 (segment (start 111.29 73.75) (end 118.3 80.76) (width 0.5) (layer B.Cu) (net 44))
 (segment (start 104.2 72.365) (end 102.365 72.365) (width 0.5) (layer B.Cu) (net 45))
 (segment (start 114.26 59.8) (end 118.3 55.76) (width 0.5) (layer B.Cu) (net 45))
 (segment (start 103.8 59.8) (end 114.26 59.8) (width 0.5) (layer B.Cu) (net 45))
 (segment (start 100.8 62.8) (end 103.8 59.8) (width 0.5) (layer B.Cu) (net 45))
 (segment (start 100.8 70.8) (end 100.8 62.8) (width 0.5) (layer B.Cu) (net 45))
 (segment (start 102.365 72.365) (end 100.8 70.8) (width 0.5) (layer B.Cu) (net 45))
 (segment (start 158.88 73.8) (end 158.88 73.72) (width 0.25) (layer B.Cu) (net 4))
 (segment (start 158.88 73.72) (end 162.8 69.8) (width 0.25) (layer B.Cu) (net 4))
 (segment (start 162.8 69.8) (end 170.8 69.8) (width 0.25) (layer B.Cu) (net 4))
 (segment (start 170.8 69.8) (end 173.8 66.8) (width 0.25) (layer B.Cu) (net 4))
 (segment (start 143.8 80.85) (end 143.8 65.8) (width 1.5) (layer B.Cu) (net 42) (status 400000))
 (segment (start 143.8 65.8) (end 151.8 57.8) (width 1.5) (layer B.Cu) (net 42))
 (segment (start 143.8 80.85) (end 143.8 80.8) (width 1.5) (layer B.Cu) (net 42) (status C00000))
 (segment (start 148.8 60.8) (end 151.8 57.8) (width 1.5) (layer B.Cu) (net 42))
 (segment (start 171.8 53.8) (end 178.8 46.8) (width 1.5) (layer B.Cu) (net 42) (status 800000))
 (segment (start 151.8 57.8) (end 155.8 53.8) (width 1.5) (layer B.Cu) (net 42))
 (segment (start 155.8 53.8) (end 171.8 53.8) (width 1.5) (layer B.Cu) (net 42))
 (segment (start 106.8 91.8) (end 132.85 91.8) (width 1.5) (layer B.Cu) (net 42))
 (segment (start 132.85 91.8) (end 143.8 80.85) (width 1.5) (layer B.Cu) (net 42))
 (segment (start 101.8 106.3) (end 104.3 106.3) (width 1.5) (layer B.Cu) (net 42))
 (segment (start 106.8 103.8) (end 106.8 91.8) (width 1.5) (layer B.Cu) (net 42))
 (segment (start 104.3 106.3) (end 106.8 103.8) (width 1.5) (layer B.Cu) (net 42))
 (segment (start 143.8 55.8) (end 132.8 66.8) (width 1.5) (layer B.Cu) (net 43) (status 400000))
 (segment (start 132.8 82.8) (end 131.8 83.8) (width 1.5) (layer B.Cu) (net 43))
 (segment (start 132.8 66.8) (end 132.8 82.8) (width 1.5) (layer B.Cu) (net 43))
 (segment (start 143.8 55.8) (end 152.8 46.8) (width 1.5) (layer B.Cu) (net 43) (status 400000))
 (segment (start 152.8 46.8) (end 158.8 46.8) (width 1.5) (layer B.Cu) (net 43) (status 800000))
 (segment (start 99.3 90.4) (end 99.3 90.3) (width 1.5) (layer B.Cu) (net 43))
 (segment (start 99.3 90.3) (end 102.8 86.8) (width 1.5) (layer B.Cu) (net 43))
 (segment (start 102.8 86.8) (end 128.8 86.8) (width 1.5) (layer B.Cu) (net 43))
 (segment (start 128.8 86.8) (end 131.8 83.8) (width 1.5) (layer B.Cu) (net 43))
 (segment (start 101.8 98.8) (end 101.8 96.8) (width 1.5) (layer B.Cu) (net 43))
 (segment (start 99.3 94.3) (end 99.3 90.4) (width 1.5) (layer B.Cu) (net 43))
 (segment (start 101.8 96.8) (end 99.3 94.3) (width 1.5) (layer B.Cu) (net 43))
 (segment (start 153.8 78.88) (end 153.8 78.8) (width 0.25) (layer B.Cu) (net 5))
 (segment (start 153.8 78.8) (end 156.8 75.8) (width 0.25) (layer B.Cu) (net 5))
 (segment (start 156.8 75.8) (end 156.8 72.8) (width 0.25) (layer B.Cu) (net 5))
 (segment (start 156.8 72.8) (end 158.8 70.8) (width 0.25) (layer B.Cu) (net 5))
 (segment (start 158.8 70.8) (end 159.8 70.8) (width 0.25) (layer B.Cu) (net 5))
 (segment (start 159.8 70.8) (end 163.8 66.8) (width 0.25) (layer B.Cu) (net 5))
 (segment (start 118.3 75.76) (end 118.3 60.76) (width 0.25) (layer B.Cu) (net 46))
 (segment (start 118.3 75.76) (end 118.84 75.76) (width 0.25) (layer B.Cu) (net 46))
 (segment (start 107.15 135.74) (end 106.74 135.74) (width 0.25) (layer B.Cu) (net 24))
 (segment (start 106.74 135.74) (end 102.8 131.8) (width 0.25) (layer B.Cu) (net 24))
 (segment (start 102.8 131.8) (end 102.8 112.8) (width 0.25) (layer B.Cu) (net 24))
 (via (at 102.8 112.8) (size 0.6) (drill 0.4) (layers F.Cu B.Cu) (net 24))
 (segment (start 102.8 112.8) (end 108.8 106.8) (width 0.25) (layer F.Cu) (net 24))
 (segment (start 108.8 106.8) (end 108.8 65.8) (width 0.25) (layer F.Cu) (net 24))
 (via (at 108.8 65.8) (size 0.6) (drill 0.4) (layers F.Cu B.Cu) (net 24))
 (segment (start 108.8 65.8) (end 108.8 63.8) (width 0.25) (layer B.Cu) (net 24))
 (segment (start 108.8 63.8) (end 107.67 62.67) (width 0.25) (layer B.Cu) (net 24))
 (segment (start 107.67 62.67) (end 106.74 62.67) (width 0.25) (layer B.Cu) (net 24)))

